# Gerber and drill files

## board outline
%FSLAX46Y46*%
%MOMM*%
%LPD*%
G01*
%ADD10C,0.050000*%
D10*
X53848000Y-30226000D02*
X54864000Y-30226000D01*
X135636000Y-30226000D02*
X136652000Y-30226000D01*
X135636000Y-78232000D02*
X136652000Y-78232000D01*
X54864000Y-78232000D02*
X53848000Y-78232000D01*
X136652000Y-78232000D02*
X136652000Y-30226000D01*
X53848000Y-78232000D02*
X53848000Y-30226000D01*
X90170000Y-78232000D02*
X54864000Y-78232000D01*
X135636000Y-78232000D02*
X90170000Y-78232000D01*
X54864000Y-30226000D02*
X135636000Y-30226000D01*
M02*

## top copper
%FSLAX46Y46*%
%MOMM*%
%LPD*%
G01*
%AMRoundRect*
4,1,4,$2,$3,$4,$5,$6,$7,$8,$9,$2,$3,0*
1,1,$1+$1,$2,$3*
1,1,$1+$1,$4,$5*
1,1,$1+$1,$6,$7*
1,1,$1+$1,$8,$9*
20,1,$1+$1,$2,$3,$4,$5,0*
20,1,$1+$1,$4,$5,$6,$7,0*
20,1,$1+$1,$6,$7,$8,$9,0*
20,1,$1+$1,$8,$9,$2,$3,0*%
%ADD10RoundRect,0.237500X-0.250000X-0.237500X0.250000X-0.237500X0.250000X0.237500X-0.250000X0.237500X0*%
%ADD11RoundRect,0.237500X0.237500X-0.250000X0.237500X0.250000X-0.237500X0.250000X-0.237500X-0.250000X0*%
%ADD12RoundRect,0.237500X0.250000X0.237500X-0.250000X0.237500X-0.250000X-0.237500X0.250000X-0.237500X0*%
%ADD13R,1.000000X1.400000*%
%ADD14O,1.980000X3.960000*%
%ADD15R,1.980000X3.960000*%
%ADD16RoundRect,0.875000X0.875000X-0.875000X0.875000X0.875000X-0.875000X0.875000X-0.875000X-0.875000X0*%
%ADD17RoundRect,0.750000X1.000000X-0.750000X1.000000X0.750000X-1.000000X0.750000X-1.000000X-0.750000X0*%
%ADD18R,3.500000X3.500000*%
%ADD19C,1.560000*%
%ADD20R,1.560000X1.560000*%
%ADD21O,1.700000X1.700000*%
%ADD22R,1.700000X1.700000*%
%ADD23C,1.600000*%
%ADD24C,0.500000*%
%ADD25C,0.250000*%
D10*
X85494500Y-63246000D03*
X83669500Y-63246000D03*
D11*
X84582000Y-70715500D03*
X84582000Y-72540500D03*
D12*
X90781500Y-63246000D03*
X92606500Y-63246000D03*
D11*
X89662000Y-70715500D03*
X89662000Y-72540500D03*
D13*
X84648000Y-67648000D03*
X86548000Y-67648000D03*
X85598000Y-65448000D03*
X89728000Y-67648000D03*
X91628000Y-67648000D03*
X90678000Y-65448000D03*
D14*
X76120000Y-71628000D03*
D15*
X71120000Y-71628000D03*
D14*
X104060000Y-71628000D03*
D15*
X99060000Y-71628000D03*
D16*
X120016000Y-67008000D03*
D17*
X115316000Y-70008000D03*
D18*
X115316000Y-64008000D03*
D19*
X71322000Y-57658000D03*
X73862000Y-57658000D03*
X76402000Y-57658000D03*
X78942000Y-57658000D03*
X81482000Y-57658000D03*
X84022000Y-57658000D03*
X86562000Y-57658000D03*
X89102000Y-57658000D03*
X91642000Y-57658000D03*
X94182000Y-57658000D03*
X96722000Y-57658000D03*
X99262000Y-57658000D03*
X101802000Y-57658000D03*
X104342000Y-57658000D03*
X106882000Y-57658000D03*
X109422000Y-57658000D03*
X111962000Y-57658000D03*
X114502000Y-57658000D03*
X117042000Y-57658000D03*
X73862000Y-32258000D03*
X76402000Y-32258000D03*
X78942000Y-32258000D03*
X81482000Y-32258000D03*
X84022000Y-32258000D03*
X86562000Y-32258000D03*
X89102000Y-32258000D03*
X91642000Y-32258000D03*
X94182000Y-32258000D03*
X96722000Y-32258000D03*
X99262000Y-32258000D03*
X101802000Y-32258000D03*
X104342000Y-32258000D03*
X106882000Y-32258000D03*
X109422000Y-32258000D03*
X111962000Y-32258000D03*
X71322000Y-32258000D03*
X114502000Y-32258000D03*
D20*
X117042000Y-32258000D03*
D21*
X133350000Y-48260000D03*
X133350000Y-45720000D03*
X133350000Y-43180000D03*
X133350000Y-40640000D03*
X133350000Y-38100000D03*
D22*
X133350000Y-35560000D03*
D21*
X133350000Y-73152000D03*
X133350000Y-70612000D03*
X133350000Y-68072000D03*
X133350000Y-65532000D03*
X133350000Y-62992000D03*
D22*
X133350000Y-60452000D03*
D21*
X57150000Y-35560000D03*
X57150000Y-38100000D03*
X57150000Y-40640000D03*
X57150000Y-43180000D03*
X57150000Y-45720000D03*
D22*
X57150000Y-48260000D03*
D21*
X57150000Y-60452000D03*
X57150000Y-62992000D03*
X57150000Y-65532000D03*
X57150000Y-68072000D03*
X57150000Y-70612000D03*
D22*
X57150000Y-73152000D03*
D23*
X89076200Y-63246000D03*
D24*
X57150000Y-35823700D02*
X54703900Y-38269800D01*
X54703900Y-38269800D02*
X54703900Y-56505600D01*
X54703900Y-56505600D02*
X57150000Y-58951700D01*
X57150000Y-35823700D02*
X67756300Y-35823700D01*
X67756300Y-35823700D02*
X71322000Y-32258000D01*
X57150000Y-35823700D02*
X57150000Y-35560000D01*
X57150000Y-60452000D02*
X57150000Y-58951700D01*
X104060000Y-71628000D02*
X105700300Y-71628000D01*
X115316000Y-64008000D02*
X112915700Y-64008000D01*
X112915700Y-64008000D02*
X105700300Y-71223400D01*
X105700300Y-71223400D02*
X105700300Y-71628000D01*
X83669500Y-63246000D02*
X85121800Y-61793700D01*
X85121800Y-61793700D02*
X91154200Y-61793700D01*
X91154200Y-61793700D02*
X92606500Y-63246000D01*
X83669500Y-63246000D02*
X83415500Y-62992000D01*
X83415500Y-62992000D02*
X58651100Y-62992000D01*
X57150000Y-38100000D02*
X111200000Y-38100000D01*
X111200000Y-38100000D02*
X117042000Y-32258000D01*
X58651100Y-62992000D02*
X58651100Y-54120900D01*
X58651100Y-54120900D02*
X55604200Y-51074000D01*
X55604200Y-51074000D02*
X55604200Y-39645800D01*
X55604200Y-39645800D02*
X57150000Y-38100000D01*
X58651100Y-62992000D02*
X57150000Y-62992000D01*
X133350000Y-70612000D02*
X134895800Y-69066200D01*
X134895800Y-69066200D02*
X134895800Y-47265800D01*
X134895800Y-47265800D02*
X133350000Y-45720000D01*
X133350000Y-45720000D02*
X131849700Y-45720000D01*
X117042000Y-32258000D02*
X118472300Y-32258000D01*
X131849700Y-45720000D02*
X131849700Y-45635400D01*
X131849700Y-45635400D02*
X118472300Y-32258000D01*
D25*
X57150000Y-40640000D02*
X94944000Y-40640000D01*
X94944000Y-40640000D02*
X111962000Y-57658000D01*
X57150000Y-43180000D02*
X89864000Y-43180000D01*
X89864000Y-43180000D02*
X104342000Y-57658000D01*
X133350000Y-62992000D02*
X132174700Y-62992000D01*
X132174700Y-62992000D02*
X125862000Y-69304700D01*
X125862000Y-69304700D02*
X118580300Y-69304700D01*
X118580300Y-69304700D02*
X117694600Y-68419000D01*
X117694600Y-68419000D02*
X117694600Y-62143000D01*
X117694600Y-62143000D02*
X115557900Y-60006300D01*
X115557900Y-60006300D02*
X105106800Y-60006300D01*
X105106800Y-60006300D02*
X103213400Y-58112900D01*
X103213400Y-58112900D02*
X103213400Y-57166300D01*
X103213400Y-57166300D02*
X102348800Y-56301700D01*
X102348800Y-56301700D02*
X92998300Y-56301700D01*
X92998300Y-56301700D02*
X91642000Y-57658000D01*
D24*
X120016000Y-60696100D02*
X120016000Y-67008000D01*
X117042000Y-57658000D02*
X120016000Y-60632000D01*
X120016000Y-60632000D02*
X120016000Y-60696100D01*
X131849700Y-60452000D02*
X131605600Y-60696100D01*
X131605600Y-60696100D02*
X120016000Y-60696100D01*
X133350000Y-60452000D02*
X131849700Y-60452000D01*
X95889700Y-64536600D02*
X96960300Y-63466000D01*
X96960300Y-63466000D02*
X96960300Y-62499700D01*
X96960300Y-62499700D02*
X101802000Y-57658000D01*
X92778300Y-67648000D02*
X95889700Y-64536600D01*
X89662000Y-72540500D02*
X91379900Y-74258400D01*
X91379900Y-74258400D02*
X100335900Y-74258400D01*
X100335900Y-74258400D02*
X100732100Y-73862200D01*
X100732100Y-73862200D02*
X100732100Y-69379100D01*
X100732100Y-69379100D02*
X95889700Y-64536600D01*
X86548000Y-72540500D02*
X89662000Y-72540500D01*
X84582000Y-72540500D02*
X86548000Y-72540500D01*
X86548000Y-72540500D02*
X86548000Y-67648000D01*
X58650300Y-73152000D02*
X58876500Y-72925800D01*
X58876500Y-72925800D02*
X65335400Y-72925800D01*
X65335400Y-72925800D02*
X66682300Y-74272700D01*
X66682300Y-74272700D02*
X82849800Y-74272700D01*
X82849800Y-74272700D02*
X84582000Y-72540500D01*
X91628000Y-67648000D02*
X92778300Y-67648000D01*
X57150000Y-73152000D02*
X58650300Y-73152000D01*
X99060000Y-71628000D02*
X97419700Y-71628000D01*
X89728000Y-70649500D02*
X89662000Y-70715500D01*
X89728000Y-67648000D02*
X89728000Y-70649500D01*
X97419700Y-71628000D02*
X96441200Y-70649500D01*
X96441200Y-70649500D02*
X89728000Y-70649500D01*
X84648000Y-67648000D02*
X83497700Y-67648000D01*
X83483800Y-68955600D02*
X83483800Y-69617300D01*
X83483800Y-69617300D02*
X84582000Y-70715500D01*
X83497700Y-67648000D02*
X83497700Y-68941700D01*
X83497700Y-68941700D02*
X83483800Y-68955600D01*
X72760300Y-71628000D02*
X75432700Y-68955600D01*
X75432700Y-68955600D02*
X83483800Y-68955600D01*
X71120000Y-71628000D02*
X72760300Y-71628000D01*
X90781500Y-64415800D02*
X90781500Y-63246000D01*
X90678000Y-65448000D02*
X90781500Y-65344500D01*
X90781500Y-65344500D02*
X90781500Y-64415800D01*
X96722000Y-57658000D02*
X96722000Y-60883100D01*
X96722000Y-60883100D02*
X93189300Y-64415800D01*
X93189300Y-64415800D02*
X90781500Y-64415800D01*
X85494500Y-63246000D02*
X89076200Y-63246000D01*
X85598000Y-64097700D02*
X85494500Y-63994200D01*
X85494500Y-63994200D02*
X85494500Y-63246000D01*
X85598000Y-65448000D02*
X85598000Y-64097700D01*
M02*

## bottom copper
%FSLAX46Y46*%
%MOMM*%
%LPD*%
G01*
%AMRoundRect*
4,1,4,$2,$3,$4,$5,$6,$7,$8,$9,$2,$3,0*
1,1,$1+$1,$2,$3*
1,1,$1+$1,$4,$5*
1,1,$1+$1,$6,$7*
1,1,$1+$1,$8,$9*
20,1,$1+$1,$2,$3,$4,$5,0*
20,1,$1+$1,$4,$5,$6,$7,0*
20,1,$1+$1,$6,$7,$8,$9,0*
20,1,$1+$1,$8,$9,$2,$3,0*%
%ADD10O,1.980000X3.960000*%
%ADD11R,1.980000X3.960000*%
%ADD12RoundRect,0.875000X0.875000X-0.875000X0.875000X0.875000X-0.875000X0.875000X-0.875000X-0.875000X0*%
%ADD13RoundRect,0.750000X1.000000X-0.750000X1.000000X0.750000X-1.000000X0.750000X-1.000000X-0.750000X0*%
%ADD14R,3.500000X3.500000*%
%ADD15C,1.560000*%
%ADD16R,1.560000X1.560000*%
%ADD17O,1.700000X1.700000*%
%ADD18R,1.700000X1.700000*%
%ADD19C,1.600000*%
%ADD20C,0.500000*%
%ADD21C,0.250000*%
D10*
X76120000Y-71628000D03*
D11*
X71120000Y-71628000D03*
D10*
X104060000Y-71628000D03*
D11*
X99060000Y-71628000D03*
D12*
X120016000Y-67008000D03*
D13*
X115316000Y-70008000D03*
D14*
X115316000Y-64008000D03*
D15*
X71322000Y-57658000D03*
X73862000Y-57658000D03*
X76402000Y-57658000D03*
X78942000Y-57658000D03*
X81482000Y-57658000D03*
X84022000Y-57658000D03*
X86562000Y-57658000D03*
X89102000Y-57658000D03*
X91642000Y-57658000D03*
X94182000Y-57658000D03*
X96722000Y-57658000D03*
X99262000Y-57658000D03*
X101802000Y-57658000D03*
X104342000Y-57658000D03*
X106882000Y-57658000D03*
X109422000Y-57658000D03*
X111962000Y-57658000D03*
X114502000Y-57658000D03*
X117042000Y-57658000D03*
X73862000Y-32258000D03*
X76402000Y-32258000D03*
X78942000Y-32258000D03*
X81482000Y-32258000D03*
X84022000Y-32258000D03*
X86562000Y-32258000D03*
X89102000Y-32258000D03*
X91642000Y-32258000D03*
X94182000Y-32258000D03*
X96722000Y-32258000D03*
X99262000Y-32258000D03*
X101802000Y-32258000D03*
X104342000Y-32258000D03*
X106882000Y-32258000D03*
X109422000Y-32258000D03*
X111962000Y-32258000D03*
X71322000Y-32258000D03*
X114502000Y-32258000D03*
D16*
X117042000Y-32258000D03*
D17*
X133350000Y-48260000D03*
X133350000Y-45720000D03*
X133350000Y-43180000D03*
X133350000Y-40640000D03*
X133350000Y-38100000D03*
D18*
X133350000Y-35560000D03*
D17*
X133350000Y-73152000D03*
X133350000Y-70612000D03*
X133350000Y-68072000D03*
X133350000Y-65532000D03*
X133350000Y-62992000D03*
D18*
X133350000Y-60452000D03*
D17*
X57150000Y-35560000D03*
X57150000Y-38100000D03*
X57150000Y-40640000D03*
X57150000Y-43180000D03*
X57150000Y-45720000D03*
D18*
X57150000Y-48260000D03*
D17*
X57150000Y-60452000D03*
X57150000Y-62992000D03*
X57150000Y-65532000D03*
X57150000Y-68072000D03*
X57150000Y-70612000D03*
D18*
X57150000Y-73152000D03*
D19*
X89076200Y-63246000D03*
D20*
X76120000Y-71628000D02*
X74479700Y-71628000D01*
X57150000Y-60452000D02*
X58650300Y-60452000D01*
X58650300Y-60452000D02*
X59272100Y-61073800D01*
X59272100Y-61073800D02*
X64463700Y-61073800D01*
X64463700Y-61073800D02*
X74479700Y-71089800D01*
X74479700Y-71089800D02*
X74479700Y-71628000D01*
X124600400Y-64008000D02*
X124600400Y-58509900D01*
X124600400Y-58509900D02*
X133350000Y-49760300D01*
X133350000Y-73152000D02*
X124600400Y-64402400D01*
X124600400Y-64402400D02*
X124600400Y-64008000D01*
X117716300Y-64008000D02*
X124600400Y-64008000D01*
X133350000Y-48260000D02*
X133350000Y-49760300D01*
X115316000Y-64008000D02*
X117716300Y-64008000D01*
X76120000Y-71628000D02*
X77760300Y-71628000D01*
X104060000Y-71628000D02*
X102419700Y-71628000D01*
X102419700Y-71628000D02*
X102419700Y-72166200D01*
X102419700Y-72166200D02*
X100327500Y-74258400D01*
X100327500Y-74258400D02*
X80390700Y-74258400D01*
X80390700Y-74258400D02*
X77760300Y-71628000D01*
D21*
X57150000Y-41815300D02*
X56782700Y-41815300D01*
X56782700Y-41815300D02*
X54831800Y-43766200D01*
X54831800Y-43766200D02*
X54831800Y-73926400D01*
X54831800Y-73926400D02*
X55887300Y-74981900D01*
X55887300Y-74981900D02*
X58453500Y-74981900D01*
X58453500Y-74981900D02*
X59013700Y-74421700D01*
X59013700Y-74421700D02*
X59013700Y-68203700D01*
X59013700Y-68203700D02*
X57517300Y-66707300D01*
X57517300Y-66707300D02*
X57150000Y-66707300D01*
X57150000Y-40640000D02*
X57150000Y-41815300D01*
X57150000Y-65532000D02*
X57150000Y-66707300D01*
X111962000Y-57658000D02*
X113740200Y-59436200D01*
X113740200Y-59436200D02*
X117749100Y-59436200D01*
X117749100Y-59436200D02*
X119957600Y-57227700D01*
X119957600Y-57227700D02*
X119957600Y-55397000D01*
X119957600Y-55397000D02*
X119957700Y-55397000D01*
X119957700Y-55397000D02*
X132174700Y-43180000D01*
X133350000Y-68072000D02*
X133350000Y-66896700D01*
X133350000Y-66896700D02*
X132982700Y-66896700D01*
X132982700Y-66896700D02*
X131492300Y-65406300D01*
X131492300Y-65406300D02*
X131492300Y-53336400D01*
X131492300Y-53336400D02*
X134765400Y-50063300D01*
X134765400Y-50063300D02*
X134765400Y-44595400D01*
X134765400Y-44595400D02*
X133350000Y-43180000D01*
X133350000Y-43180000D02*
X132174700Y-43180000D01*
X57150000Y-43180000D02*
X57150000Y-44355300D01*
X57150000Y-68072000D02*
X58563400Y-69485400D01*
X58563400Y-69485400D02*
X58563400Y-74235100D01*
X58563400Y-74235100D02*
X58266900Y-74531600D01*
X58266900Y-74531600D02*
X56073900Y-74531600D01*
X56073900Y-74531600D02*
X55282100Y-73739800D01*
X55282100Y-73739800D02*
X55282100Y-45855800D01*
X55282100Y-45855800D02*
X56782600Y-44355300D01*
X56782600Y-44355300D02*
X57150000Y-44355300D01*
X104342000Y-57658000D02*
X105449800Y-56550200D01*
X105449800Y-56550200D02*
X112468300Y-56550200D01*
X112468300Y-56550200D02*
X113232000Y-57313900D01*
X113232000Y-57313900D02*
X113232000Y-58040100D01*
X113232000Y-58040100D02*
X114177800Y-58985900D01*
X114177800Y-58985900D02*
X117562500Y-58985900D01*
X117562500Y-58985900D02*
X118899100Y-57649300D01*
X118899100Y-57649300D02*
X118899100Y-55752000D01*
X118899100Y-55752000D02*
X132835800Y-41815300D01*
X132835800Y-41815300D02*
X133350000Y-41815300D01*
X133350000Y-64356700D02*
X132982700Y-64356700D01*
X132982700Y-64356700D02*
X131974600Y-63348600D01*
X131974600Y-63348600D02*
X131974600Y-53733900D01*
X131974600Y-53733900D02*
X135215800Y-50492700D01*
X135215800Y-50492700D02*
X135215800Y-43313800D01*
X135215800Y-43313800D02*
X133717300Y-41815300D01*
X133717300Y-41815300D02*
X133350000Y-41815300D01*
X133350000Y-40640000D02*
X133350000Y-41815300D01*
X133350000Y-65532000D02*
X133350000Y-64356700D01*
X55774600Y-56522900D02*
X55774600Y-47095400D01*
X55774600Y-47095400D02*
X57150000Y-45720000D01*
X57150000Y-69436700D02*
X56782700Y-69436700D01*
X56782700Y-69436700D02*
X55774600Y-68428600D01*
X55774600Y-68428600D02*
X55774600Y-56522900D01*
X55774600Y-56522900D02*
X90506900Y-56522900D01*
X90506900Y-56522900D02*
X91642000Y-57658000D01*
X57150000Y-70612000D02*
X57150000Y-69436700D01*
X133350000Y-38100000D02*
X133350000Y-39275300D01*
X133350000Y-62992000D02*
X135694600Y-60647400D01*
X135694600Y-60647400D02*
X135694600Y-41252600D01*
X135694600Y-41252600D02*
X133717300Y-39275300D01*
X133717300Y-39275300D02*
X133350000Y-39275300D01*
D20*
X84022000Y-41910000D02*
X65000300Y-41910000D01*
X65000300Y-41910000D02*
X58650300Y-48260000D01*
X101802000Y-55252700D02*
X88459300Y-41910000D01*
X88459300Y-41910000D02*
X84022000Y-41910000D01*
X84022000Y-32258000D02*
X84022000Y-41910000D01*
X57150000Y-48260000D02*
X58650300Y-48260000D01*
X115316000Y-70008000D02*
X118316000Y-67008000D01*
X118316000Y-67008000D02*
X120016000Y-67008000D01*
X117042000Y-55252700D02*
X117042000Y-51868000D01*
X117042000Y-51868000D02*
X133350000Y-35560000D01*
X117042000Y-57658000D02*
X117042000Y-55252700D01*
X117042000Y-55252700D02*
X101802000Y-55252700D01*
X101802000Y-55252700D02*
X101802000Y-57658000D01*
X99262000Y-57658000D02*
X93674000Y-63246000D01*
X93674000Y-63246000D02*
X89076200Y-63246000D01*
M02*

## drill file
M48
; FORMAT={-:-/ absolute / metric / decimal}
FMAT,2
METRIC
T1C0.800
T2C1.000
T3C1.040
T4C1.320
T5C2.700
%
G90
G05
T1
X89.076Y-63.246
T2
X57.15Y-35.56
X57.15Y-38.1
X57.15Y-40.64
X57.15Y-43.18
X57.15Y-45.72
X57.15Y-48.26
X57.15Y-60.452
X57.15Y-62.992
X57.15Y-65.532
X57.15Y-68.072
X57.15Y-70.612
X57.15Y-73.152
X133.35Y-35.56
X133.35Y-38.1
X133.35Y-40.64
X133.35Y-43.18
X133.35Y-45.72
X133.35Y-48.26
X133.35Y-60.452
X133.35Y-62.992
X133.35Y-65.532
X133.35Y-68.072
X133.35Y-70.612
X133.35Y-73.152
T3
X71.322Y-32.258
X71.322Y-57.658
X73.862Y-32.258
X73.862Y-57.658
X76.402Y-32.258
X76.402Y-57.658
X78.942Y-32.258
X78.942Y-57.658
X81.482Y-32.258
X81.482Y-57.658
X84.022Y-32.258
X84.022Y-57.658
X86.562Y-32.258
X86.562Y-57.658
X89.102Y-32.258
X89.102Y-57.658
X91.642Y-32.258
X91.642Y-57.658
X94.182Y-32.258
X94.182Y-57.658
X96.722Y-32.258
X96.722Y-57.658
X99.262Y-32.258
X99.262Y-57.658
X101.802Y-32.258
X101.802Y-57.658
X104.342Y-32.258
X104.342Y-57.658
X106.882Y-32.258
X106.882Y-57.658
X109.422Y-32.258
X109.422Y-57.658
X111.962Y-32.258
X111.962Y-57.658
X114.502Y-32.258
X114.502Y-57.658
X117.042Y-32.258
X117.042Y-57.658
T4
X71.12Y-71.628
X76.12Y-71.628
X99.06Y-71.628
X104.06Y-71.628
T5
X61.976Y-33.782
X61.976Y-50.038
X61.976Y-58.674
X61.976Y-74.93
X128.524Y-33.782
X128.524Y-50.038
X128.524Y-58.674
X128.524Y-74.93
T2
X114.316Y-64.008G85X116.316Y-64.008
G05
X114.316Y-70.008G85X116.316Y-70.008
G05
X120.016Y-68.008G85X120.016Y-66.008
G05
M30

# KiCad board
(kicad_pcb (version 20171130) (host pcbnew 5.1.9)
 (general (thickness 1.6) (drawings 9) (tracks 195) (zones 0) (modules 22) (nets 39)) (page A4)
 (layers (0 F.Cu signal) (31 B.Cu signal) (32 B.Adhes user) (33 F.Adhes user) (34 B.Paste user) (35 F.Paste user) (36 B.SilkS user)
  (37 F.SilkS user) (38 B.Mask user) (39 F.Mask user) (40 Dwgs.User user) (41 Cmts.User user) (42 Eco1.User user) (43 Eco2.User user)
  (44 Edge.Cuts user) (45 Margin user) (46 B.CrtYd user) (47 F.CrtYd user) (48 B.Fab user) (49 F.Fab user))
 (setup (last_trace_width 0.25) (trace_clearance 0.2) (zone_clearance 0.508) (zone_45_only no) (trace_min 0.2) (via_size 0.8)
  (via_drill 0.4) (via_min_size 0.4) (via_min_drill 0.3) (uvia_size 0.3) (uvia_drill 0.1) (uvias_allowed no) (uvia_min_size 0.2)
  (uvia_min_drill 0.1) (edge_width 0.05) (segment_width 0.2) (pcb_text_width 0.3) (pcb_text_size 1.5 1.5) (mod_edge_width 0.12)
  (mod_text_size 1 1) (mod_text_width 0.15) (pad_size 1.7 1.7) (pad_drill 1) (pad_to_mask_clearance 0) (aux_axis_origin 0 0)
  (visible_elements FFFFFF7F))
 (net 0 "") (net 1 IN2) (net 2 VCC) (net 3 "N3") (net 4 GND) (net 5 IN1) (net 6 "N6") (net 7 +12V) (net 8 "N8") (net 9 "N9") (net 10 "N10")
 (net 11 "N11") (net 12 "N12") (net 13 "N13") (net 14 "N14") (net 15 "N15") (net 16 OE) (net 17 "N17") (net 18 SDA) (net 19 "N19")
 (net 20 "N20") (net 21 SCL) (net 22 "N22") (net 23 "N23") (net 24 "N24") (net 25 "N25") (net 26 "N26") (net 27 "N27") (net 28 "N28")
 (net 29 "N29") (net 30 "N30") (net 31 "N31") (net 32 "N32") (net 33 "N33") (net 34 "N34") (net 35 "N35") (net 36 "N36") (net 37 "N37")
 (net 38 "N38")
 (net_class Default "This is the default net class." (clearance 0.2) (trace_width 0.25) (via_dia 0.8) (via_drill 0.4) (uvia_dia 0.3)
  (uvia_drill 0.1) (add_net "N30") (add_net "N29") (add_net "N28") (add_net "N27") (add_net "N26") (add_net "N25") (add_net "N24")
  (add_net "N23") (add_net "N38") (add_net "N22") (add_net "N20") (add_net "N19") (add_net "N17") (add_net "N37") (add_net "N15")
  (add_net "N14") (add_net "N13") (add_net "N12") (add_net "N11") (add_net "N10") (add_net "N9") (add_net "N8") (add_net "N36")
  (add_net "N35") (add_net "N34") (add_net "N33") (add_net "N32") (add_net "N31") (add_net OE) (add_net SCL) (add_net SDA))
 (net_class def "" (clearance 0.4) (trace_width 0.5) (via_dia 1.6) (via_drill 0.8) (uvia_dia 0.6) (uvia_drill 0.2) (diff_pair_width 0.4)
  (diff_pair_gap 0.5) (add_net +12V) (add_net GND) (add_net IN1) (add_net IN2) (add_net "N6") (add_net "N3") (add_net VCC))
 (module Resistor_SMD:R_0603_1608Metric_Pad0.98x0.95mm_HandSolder (layer F.Cu) (at 84.582 63.246)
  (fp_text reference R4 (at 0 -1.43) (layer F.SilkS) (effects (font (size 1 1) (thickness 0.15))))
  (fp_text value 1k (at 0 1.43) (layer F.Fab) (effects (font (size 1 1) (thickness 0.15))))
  (pad 2 smd roundrect (at 0.9125 0) (size 0.975 0.95) (layers F.Cu F.Paste F.Mask) (roundrect_rratio 0.25) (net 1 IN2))
  (pad 1 smd roundrect (at -0.9125 0) (size 0.975 0.95) (layers F.Cu F.Paste F.Mask) (roundrect_rratio 0.25) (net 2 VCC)))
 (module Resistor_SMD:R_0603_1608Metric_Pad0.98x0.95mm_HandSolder (layer F.Cu) (at 84.582 71.628 90)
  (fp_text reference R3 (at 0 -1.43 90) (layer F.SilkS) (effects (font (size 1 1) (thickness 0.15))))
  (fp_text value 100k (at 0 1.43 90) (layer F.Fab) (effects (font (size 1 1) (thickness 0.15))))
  (pad 2 smd roundrect (at 0.9125 0 90) (size 0.975 0.95) (layers F.Cu F.Paste F.Mask) (roundrect_rratio 0.25) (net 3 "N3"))
  (pad 1 smd roundrect (at -0.9125 0 90) (size 0.975 0.95) (layers F.Cu F.Paste F.Mask) (roundrect_rratio 0.25) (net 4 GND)))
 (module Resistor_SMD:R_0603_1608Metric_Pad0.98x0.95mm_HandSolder (layer F.Cu) (at 91.694 63.246 180)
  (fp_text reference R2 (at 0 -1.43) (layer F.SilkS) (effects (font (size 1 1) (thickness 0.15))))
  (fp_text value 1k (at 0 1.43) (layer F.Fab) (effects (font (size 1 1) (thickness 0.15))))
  (pad 2 smd roundrect (at 0.9125 0 180) (size 0.975 0.95) (layers F.Cu F.Paste F.Mask) (roundrect_rratio 0.25) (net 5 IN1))
  (pad 1 smd roundrect (at -0.9125 0 180) (size 0.975 0.95) (layers F.Cu F.Paste F.Mask) (roundrect_rratio 0.25) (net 2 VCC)))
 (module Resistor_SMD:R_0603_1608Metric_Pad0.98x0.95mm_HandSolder (layer F.Cu) (at 89.662 71.628 90)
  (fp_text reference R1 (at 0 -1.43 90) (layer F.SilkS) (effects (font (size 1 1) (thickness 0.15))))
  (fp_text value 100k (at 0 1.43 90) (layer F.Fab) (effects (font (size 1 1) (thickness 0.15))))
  (pad 2 smd roundrect (at 0.9125 0 90) (size 0.975 0.95) (layers F.Cu F.Paste F.Mask) (roundrect_rratio 0.25) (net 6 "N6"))
  (pad 1 smd roundrect (at -0.9125 0 90) (size 0.975 0.95) (layers F.Cu F.Paste F.Mask) (roundrect_rratio 0.25) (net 4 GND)))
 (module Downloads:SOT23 (layer F.Cu) (at 85.598 66.548)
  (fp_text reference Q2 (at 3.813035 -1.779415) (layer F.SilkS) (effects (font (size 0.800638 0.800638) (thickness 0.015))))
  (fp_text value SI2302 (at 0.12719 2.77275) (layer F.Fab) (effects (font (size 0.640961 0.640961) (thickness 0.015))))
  (pad 1 smd rect (at -0.95 1.1) (size 1 1.4) (layers F.Cu F.Paste F.Mask) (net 3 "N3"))
  (pad 2 smd rect (at 0.95 1.1) (size 1 1.4) (layers F.Cu F.Paste F.Mask) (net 4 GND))
  (pad 3 smd rect (at 0 -1.1) (size 1 1.4) (layers F.Cu F.Paste F.Mask) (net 1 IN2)))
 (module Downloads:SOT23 (layer F.Cu) (at 90.678 66.548)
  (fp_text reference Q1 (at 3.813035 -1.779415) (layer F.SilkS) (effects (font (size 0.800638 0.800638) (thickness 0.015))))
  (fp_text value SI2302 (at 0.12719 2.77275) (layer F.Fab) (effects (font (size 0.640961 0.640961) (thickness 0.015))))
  (pad 1 smd rect (at -0.95 1.1) (size 1 1.4) (layers F.Cu F.Paste F.Mask) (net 6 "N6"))
  (pad 2 smd rect (at 0.95 1.1) (size 1 1.4) (layers F.Cu F.Paste F.Mask) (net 4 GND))
  (pad 3 smd rect (at 0 -1.1) (size 1 1.4) (layers F.Cu F.Paste F.Mask) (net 5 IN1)))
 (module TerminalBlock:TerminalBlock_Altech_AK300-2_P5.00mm (layer F.Cu) (at 71.12 71.628)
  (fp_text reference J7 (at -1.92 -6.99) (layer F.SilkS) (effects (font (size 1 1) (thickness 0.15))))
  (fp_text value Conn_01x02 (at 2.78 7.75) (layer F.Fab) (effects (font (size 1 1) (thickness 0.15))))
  (pad 2 thru_hole oval (at 5 0) (size 1.98 3.96) (drill 1.32) (layers *.Cu *.Mask) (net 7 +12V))
  (pad 1 thru_hole rect (at 0 0) (size 1.98 3.96) (drill 1.32) (layers *.Cu *.Mask) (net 3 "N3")))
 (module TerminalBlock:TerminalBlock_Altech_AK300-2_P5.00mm (layer F.Cu) (at 99.06 71.628)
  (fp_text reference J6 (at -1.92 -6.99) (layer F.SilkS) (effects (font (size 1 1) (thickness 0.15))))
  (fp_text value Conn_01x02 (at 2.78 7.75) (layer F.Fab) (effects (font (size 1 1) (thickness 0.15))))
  (pad 2 thru_hole oval (at 5 0) (size 1.98 3.96) (drill 1.32) (layers *.Cu *.Mask) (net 7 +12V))
  (pad 1 thru_hole rect (at 0 0) (size 1.98 3.96) (drill 1.32) (layers *.Cu *.Mask) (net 6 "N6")))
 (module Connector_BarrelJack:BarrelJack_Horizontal (layer F.Cu) (at 115.316 64.008 90)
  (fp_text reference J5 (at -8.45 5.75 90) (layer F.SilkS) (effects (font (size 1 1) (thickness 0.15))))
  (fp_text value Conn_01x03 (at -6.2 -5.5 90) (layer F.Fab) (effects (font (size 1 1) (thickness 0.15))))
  (pad 3 thru_hole roundrect (at -3 4.7 90) (size 3.5 3.5) (drill oval 3 1) (layers *.Cu *.Mask) (roundrect_rratio 0.25) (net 4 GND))
  (pad 2 thru_hole roundrect (at -6 0 90) (size 3 3.5) (drill oval 1 3) (layers *.Cu *.Mask) (roundrect_rratio 0.25) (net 4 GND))
  (pad 1 thru_hole rect (at 0 0 90) (size 3.5 3.5) (drill oval 1 3) (layers *.Cu *.Mask) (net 7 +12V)))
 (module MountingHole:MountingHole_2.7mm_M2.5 (layer F.Cu) (at 128.524 74.93)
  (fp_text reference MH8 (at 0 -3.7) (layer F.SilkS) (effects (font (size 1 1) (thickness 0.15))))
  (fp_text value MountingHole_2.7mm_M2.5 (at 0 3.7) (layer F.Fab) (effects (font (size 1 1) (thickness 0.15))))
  (pad 1 np_thru_hole circle (at 0 0) (size 2.7 2.7) (drill 2.7) (layers *.Cu *.Mask)))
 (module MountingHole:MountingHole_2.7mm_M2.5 (layer F.Cu) (at 128.524 58.674)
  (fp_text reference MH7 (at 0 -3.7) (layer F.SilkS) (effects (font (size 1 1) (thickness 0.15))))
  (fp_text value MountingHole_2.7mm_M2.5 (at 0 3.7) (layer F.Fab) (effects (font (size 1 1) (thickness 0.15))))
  (pad 1 np_thru_hole circle (at 0 0) (size 2.7 2.7) (drill 2.7) (layers *.Cu *.Mask)))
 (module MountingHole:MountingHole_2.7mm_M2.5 (layer F.Cu) (at 128.524 50.038)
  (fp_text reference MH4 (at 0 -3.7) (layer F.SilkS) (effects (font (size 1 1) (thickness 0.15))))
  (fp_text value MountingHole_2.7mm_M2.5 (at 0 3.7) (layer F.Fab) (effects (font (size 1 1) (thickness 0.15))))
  (pad 1 np_thru_hole circle (at 0 0) (size 2.7 2.7) (drill 2.7) (layers *.Cu *.Mask)))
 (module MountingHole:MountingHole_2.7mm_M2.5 (layer F.Cu) (at 128.524 33.782)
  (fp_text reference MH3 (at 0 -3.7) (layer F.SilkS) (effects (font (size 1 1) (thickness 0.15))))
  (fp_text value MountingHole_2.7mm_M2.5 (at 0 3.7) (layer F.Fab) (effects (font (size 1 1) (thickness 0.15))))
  (pad 1 np_thru_hole circle (at 0 0) (size 2.7 2.7) (drill 2.7) (layers *.Cu *.Mask)))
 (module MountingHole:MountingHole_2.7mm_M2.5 (layer F.Cu) (at 61.976 74.93)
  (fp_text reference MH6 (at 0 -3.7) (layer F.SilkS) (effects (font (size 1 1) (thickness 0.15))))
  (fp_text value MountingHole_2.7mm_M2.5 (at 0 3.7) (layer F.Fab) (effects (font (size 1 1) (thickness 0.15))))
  (pad 1 np_thru_hole circle (at 0 0) (size 2.7 2.7) (drill 2.7) (layers *.Cu *.Mask)))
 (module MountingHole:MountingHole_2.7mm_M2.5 (layer F.Cu) (at 61.976 58.674)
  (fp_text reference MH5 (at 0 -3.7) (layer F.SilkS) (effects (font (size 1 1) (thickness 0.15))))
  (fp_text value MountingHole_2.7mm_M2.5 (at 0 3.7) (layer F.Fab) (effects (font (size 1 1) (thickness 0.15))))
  (pad 1 np_thru_hole circle (at 0 0) (size 2.7 2.7) (drill 2.7) (layers *.Cu *.Mask)))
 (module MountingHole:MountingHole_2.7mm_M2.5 (layer F.Cu) (at 61.976 50.038)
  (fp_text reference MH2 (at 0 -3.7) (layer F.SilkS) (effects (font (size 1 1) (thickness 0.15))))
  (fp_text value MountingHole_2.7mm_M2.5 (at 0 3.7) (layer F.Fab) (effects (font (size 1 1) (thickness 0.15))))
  (pad 1 np_thru_hole circle (at 0 0) (size 2.7 2.7) (drill 2.7) (layers *.Cu *.Mask)))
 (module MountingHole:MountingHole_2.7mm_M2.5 (layer F.Cu) (at 61.976 33.782)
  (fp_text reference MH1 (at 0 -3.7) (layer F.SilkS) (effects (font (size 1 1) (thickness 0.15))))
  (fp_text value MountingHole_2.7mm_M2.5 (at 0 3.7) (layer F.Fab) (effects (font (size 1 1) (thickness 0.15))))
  (pad 1 np_thru_hole circle (at 0 0) (size 2.7 2.7) (drill 2.7) (layers *.Cu *.Mask)))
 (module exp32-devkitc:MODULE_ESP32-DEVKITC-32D (layer F.Cu) (at 97.282 44.958 270)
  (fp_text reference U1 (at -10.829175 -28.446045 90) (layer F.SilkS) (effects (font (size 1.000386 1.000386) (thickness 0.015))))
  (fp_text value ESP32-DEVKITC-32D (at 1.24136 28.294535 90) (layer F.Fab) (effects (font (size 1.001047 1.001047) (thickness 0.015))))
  (pad 38 thru_hole circle (at 12.7 25.96 270) (size 1.56 1.56) (drill 1.04) (layers *.Cu *.Mask) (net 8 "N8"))
  (pad 37 thru_hole circle (at 12.7 23.42 270) (size 1.56 1.56) (drill 1.04) (layers *.Cu *.Mask) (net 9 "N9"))
  (pad 36 thru_hole circle (at 12.7 20.88 270) (size 1.56 1.56) (drill 1.04) (layers *.Cu *.Mask) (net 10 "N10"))
  (pad 35 thru_hole circle (at 12.7 18.34 270) (size 1.56 1.56) (drill 1.04) (layers *.Cu *.Mask) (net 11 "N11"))
  (pad 34 thru_hole circle (at 12.7 15.8 270) (size 1.56 1.56) (drill 1.04) (layers *.Cu *.Mask) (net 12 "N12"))
  (pad 33 thru_hole circle (at 12.7 13.26 270) (size 1.56 1.56) (drill 1.04) (layers *.Cu *.Mask) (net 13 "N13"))
  (pad 32 thru_hole circle (at 12.7 10.72 270) (size 1.56 1.56) (drill 1.04) (layers *.Cu *.Mask) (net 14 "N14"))
  (pad 31 thru_hole circle (at 12.7 8.18 270) (size 1.56 1.56) (drill 1.04) (layers *.Cu *.Mask) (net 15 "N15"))
  (pad 30 thru_hole circle (at 12.7 5.64 270) (size 1.56 1.56) (drill 1.04) (layers *.Cu *.Mask) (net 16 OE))
  (pad 29 thru_hole circle (at 12.7 3.1 270) (size 1.56 1.56) (drill 1.04) (layers *.Cu *.Mask) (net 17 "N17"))
  (pad 28 thru_hole circle (at 12.7 0.56 270) (size 1.56 1.56) (drill 1.04) (layers *.Cu *.Mask) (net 5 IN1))
  (pad 27 thru_hole circle (at 12.7 -1.98 270) (size 1.56 1.56) (drill 1.04) (layers *.Cu *.Mask) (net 1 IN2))
  (pad 26 thru_hole circle (at 12.7 -4.52 270) (size 1.56 1.56) (drill 1.04) (layers *.Cu *.Mask) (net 4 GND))
  (pad 25 thru_hole circle (at 12.7 -7.06 270) (size 1.56 1.56) (drill 1.04) (layers *.Cu *.Mask) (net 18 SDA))
  (pad 24 thru_hole circle (at 12.7 -9.6 270) (size 1.56 1.56) (drill 1.04) (layers *.Cu *.Mask) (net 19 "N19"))
  (pad 23 thru_hole circle (at 12.7 -12.14 270) (size 1.56 1.56) (drill 1.04) (layers *.Cu *.Mask) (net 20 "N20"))
  (pad 22 thru_hole circle (at 12.7 -14.68 270) (size 1.56 1.56) (drill 1.04) (layers *.Cu *.Mask) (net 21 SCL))
  (pad 21 thru_hole circle (at 12.7 -17.22 270) (size 1.56 1.56) (drill 1.04) (layers *.Cu *.Mask) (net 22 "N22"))
  (pad 20 thru_hole circle (at 12.7 -19.76 270) (size 1.56 1.56) (drill 1.04) (layers *.Cu *.Mask) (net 4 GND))
  (pad 18 thru_hole circle (at -12.7 23.42 270) (size 1.56 1.56) (drill 1.04) (layers *.Cu *.Mask) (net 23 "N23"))
  (pad 17 thru_hole circle (at -12.7 20.88 270) (size 1.56 1.56) (drill 1.04) (layers *.Cu *.Mask) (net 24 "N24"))
  (pad 16 thru_hole circle (at -12.7 18.34 270) (size 1.56 1.56) (drill 1.04) (layers *.Cu *.Mask) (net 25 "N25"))
  (pad 15 thru_hole circle (at -12.7 15.8 270) (size 1.56 1.56) (drill 1.04) (layers *.Cu *.Mask) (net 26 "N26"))
  (pad 14 thru_hole circle (at -12.7 13.26 270) (size 1.56 1.56) (drill 1.04) (layers *.Cu *.Mask) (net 4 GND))
  (pad 13 thru_hole circle (at -12.7 10.72 270) (size 1.56 1.56) (drill 1.04) (layers *.Cu *.Mask) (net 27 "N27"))
  (pad 12 thru_hole circle (at -12.7 8.18 270) (size 1.56 1.56) (drill 1.04) (layers *.Cu *.Mask) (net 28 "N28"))
  (pad 11 thru_hole circle (at -12.7 5.64 270) (size 1.56 1.56) (drill 1.04) (layers *.Cu *.Mask) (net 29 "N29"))
  (pad 10 thru_hole circle (at -12.7 3.1 270) (size 1.56 1.56) (drill 1.04) (layers *.Cu *.Mask) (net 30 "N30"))
  (pad 9 thru_hole circle (at -12.7 0.56 270) (size 1.56 1.56) (drill 1.04) (layers *.Cu *.Mask) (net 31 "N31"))
  (pad 8 thru_hole circle (at -12.7 -1.98 270) (size 1.56 1.56) (drill 1.04) (layers *.Cu *.Mask) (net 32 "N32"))
  (pad 7 thru_hole circle (at -12.7 -4.52 270) (size 1.56 1.56) (drill 1.04) (layers *.Cu *.Mask) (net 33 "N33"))
  (pad 6 thru_hole circle (at -12.7 -7.06 270) (size 1.56 1.56) (drill 1.04) (layers *.Cu *.Mask) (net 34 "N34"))
  (pad 5 thru_hole circle (at -12.7 -9.6 270) (size 1.56 1.56) (drill 1.04) (layers *.Cu *.Mask) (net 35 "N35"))
  (pad 4 thru_hole circle (at -12.7 -12.14 270) (size 1.56 1.56) (drill 1.04) (layers *.Cu *.Mask) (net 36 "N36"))
  (pad 3 thru_hole circle (at -12.7 -14.68 270) (size 1.56 1.56) (drill 1.04) (layers *.Cu *.Mask) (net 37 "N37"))
  (pad 19 thru_hole circle (at -12.7 25.96 270) (size 1.56 1.56) (drill 1.04) (layers *.Cu *.Mask) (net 7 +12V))
  (pad 2 thru_hole circle (at -12.7 -17.22 270) (size 1.56 1.56) (drill 1.04) (layers *.Cu *.Mask) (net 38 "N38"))
  (pad 1 thru_hole rect (at -12.7 -19.76 270) (size 1.56 1.56) (drill 1.04) (layers *.Cu *.Mask) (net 2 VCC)))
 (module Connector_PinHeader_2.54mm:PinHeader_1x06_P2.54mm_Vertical (layer F.Cu) (at 133.35 35.56)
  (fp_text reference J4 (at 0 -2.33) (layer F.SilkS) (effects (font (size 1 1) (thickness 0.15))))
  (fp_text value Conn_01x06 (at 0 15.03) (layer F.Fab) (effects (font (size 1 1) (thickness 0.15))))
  (pad 6 thru_hole oval (at 0 12.7) (size 1.7 1.7) (drill 1) (layers *.Cu *.Mask) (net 7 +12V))
  (pad 5 thru_hole oval (at 0 10.16) (size 1.7 1.7) (drill 1) (layers *.Cu *.Mask) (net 2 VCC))
  (pad 4 thru_hole oval (at 0 7.62) (size 1.7 1.7) (drill 1) (layers *.Cu *.Mask) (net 21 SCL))
  (pad 3 thru_hole oval (at 0 5.08) (size 1.7 1.7) (drill 1) (layers *.Cu *.Mask) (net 18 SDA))
  (pad 2 thru_hole oval (at 0 2.54) (size 1.7 1.7) (drill 1) (layers *.Cu *.Mask) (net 16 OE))
  (pad 1 thru_hole rect (at 0 0) (size 1.7 1.7) (drill 1) (layers *.Cu *.Mask) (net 4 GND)))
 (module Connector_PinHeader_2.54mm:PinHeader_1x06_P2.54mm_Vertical (layer F.Cu) (at 133.35 60.452)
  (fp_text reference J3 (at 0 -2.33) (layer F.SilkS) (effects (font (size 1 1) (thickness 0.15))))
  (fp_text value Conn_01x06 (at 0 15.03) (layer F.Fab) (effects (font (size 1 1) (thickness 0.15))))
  (pad 6 thru_hole oval (at 0 12.7) (size 1.7 1.7) (drill 1) (layers *.Cu *.Mask) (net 7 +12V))
  (pad 5 thru_hole oval (at 0 10.16) (size 1.7 1.7) (drill 1) (layers *.Cu *.Mask) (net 2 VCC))
  (pad 4 thru_hole oval (at 0 7.62) (size 1.7 1.7) (drill 1) (layers *.Cu *.Mask) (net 21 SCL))
  (pad 3 thru_hole oval (at 0 5.08) (size 1.7 1.7) (drill 1) (layers *.Cu *.Mask) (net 18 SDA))
  (pad 2 thru_hole oval (at 0 2.54) (size 1.7 1.7) (drill 1) (layers *.Cu *.Mask) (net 16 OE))
  (pad 1 thru_hole rect (at 0 0) (size 1.7 1.7) (drill 1) (layers *.Cu *.Mask) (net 4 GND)))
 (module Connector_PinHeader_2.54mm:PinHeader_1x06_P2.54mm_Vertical (layer F.Cu) (at 57.15 48.26 180)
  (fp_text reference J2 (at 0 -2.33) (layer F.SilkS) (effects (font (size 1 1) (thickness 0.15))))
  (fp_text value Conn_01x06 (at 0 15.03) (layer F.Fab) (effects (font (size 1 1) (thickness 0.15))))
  (pad 6 thru_hole oval (at 0 12.7 180) (size 1.7 1.7) (drill 1) (layers *.Cu *.Mask) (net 7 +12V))
  (pad 5 thru_hole oval (at 0 10.16 180) (size 1.7 1.7) (drill 1) (layers *.Cu *.Mask) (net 2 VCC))
  (pad 4 thru_hole oval (at 0 7.62 180) (size 1.7 1.7) (drill 1) (layers *.Cu *.Mask) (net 21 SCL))
  (pad 3 thru_hole oval (at 0 5.08 180) (size 1.7 1.7) (drill 1) (layers *.Cu *.Mask) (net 18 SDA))
  (pad 2 thru_hole oval (at 0 2.54 180) (size 1.7 1.7) (drill 1) (layers *.Cu *.Mask) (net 16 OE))
  (pad 1 thru_hole rect (at 0 0 180) (size 1.7 1.7) (drill 1) (layers *.Cu *.Mask) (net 4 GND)))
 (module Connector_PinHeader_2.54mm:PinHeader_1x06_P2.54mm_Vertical (layer F.Cu) (at 57.15 73.152 180)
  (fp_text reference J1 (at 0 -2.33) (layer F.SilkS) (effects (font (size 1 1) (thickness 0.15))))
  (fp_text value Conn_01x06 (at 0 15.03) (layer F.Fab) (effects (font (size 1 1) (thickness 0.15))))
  (pad 6 thru_hole oval (at 0 12.7 180) (size 1.7 1.7) (drill 1) (layers *.Cu *.Mask) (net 7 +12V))
  (pad 5 thru_hole oval (at 0 10.16 180) (size 1.7 1.7) (drill 1) (layers *.Cu *.Mask) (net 2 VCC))
  (pad 4 thru_hole oval (at 0 7.62 180) (size 1.7 1.7) (drill 1) (layers *.Cu *.Mask) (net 21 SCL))
  (pad 3 thru_hole oval (at 0 5.08 180) (size 1.7 1.7) (drill 1) (layers *.Cu *.Mask) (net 18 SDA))
  (pad 2 thru_hole oval (at 0 2.54 180) (size 1.7 1.7) (drill 1) (layers *.Cu *.Mask) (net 16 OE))
  (pad 1 thru_hole rect (at 0 0 180) (size 1.7 1.7) (drill 1) (layers *.Cu *.Mask) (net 4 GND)))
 (gr_line (start 53.848 30.226) (end 54.864 30.226) (layer Edge.Cuts) (width 0.05))
 (gr_line (start 135.636 30.226) (end 136.652 30.226) (layer Edge.Cuts) (width 0.05))
 (gr_line (start 135.636 78.232) (end 136.652 78.232) (layer Edge.Cuts) (width 0.05))
 (gr_line (start 54.864 78.232) (end 53.848 78.232) (layer Edge.Cuts) (width 0.05))
 (gr_line (start 136.652 78.232) (end 136.652 30.226) (layer Edge.Cuts) (width 0.05))
 (gr_line (start 53.848 78.232) (end 53.848 30.226) (layer Edge.Cuts) (width 0.05))
 (gr_line (start 90.17 78.232) (end 54.864 78.232) (layer Edge.Cuts) (width 0.05))
 (gr_line (start 135.636 78.232) (end 90.17 78.232) (layer Edge.Cuts) (width 0.05))
 (gr_line (start 54.864 30.226) (end 135.636 30.226) (layer Edge.Cuts) (width 0.05))
 (segment (start 76.12 71.628) (end 74.4797 71.628) (width 0.5) (layer B.Cu) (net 7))
 (segment (start 57.15 60.452) (end 58.6503 60.452) (width 0.5) (layer B.Cu) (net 7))
 (segment (start 58.6503 60.452) (end 59.2721 61.0738) (width 0.5) (layer B.Cu) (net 7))
 (segment (start 59.2721 61.0738) (end 64.4637 61.0738) (width 0.5) (layer B.Cu) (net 7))
 (segment (start 64.4637 61.0738) (end 74.4797 71.0898) (width 0.5) (layer B.Cu) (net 7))
 (segment (start 74.4797 71.0898) (end 74.4797 71.628) (width 0.5) (layer B.Cu) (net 7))
 (segment (start 57.15 35.8237) (end 54.7039 38.2698) (width 0.5) (layer F.Cu) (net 7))
 (segment (start 54.7039 38.2698) (end 54.7039 56.5056) (width 0.5) (layer F.Cu) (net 7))
 (segment (start 54.7039 56.5056) (end 57.15 58.9517) (width 0.5) (layer F.Cu) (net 7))
 (segment (start 124.6004 64.008) (end 124.6004 58.5099) (width 0.5) (layer B.Cu) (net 7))
 (segment (start 124.6004 58.5099) (end 133.35 49.7603) (width 0.5) (layer B.Cu) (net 7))
 (segment (start 133.35 73.152) (end 124.6004 64.4024) (width 0.5) (layer B.Cu) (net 7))
 (segment (start 124.6004 64.4024) (end 124.6004 64.008) (width 0.5) (layer B.Cu) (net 7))
 (segment (start 117.7163 64.008) (end 124.6004 64.008) (width 0.5) (layer B.Cu) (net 7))
 (segment (start 133.35 48.26) (end 133.35 49.7603) (width 0.5) (layer B.Cu) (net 7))
 (segment (start 115.316 64.008) (end 117.7163 64.008) (width 0.5) (layer B.Cu) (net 7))
 (segment (start 57.15 35.8237) (end 67.7563 35.8237) (width 0.5) (layer F.Cu) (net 7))
 (segment (start 67.7563 35.8237) (end 71.322 32.258) (width 0.5) (layer F.Cu) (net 7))
 (segment (start 57.15 35.8237) (end 57.15 35.56) (width 0.5) (layer F.Cu) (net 7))
 (segment (start 57.15 60.452) (end 57.15 58.9517) (width 0.5) (layer F.Cu) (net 7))
 (segment (start 76.12 71.628) (end 77.7603 71.628) (width 0.5) (layer B.Cu) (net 7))
 (segment (start 104.06 71.628) (end 102.4197 71.628) (width 0.5) (layer B.Cu) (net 7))
 (segment (start 102.4197 71.628) (end 102.4197 72.1662) (width 0.5) (layer B.Cu) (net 7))
 (segment (start 102.4197 72.1662) (end 100.3275 74.2584) (width 0.5) (layer B.Cu) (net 7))
 (segment (start 100.3275 74.2584) (end 80.3907 74.2584) (width 0.5) (layer B.Cu) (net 7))
 (segment (start 80.3907 74.2584) (end 77.7603 71.628) (width 0.5) (layer B.Cu) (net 7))
 (segment (start 104.06 71.628) (end 105.7003 71.628) (width 0.5) (layer F.Cu) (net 7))
 (segment (start 115.316 64.008) (end 112.9157 64.008) (width 0.5) (layer F.Cu) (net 7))
 (segment (start 112.9157 64.008) (end 105.7003 71.2234) (width 0.5) (layer F.Cu) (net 7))
 (segment (start 105.7003 71.2234) (end 105.7003 71.628) (width 0.5) (layer F.Cu) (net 7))
 (segment (start 83.6695 63.246) (end 85.1218 61.7937) (width 0.5) (layer F.Cu) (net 2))
 (segment (start 85.1218 61.7937) (end 91.1542 61.7937) (width 0.5) (layer F.Cu) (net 2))
 (segment (start 91.1542 61.7937) (end 92.6065 63.246) (width 0.5) (layer F.Cu) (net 2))
 (segment (start 83.6695 63.246) (end 83.4155 62.992) (width 0.5) (layer F.Cu) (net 2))
 (segment (start 83.4155 62.992) (end 58.6511 62.992) (width 0.5) (layer F.Cu) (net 2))
 (segment (start 57.15 38.1) (end 111.2 38.1) (width 0.5) (layer F.Cu) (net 2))
 (segment (start 111.2 38.1) (end 117.042 32.258) (width 0.5) (layer F.Cu) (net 2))
 (segment (start 58.6511 62.992) (end 58.6511 54.1209) (width 0.5) (layer F.Cu) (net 2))
 (segment (start 58.6511 54.1209) (end 55.6042 51.074) (width 0.5) (layer F.Cu) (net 2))
 (segment (start 55.6042 51.074) (end 55.6042 39.6458) (width 0.5) (layer F.Cu) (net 2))
 (segment (start 55.6042 39.6458) (end 57.15 38.1) (width 0.5) (layer F.Cu) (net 2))
 (segment (start 58.6511 62.992) (end 57.15 62.992) (width 0.5) (layer F.Cu) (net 2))
 (segment (start 133.35 70.612) (end 134.8958 69.0662) (width 0.5) (layer F.Cu) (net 2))
 (segment (start 134.8958 69.0662) (end 134.8958 47.2658) (width 0.5) (layer F.Cu) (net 2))
 (segment (start 134.8958 47.2658) (end 133.35 45.72) (width 0.5) (layer F.Cu) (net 2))
 (segment (start 133.35 45.72) (end 131.8497 45.72) (width 0.5) (layer F.Cu) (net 2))
 (segment (start 117.042 32.258) (end 118.4723 32.258) (width 0.5) (layer F.Cu) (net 2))
 (segment (start 131.8497 45.72) (end 131.8497 45.6354) (width 0.5) (layer F.Cu) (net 2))
 (segment (start 131.8497 45.6354) (end 118.4723 32.258) (width 0.5) (layer F.Cu) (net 2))
 (segment (start 57.15 41.8153) (end 56.7827 41.8153) (width 0.25) (layer B.Cu) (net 21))
 (segment (start 56.7827 41.8153) (end 54.8318 43.7662) (width 0.25) (layer B.Cu) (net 21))
 (segment (start 54.8318 43.7662) (end 54.8318 73.9264) (width 0.25) (layer B.Cu) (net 21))
 (segment (start 54.8318 73.9264) (end 55.8873 74.9819) (width 0.25) (layer B.Cu) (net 21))
 (segment (start 55.8873 74.9819) (end 58.4535 74.9819) (width 0.25) (layer B.Cu) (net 21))
 (segment (start 58.4535 74.9819) (end 59.0137 74.4217) (width 0.25) (layer B.Cu) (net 21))
 (segment (start 59.0137 74.4217) (end 59.0137 68.2037) (width 0.25) (layer B.Cu) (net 21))
 (segment (start 59.0137 68.2037) (end 57.5173 66.7073) (width 0.25) (layer B.Cu) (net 21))
 (segment (start 57.5173 66.7073) (end 57.15 66.7073) (width 0.25) (layer B.Cu) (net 21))
 (segment (start 57.15 40.64) (end 57.15 41.8153) (width 0.25) (layer B.Cu) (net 21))
 (segment (start 57.15 65.532) (end 57.15 66.7073) (width 0.25) (layer B.Cu) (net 21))
 (segment (start 111.962 57.658) (end 113.7402 59.4362) (width 0.25) (layer B.Cu) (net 21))
 (segment (start 113.7402 59.4362) (end 117.7491 59.4362) (width 0.25) (layer B.Cu) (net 21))
 (segment (start 117.7491 59.4362) (end 119.9576 57.2277) (width 0.25) (layer B.Cu) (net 21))
 (segment (start 119.9576 57.2277) (end 119.9576 55.397) (width 0.25) (layer B.Cu) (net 21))
 (segment (start 119.9576 55.397) (end 119.9577 55.397) (width 0.25) (layer B.Cu) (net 21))
 (segment (start 119.9577 55.397) (end 132.1747 43.18) (width 0.25) (layer B.Cu) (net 21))
 (segment (start 133.35 68.072) (end 133.35 66.8967) (width 0.25) (layer B.Cu) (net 21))
 (segment (start 133.35 66.8967) (end 132.9827 66.8967) (width 0.25) (layer B.Cu) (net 21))
 (segment (start 132.9827 66.8967) (end 131.4923 65.4063) (width 0.25) (layer B.Cu) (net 21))
 (segment (start 131.4923 65.4063) (end 131.4923 53.3364) (width 0.25) (layer B.Cu) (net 21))
 (segment (start 131.4923 53.3364) (end 134.7654 50.0633) (width 0.25) (layer B.Cu) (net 21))
 (segment (start 134.7654 50.0633) (end 134.7654 44.5954) (width 0.25) (layer B.Cu) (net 21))
 (segment (start 134.7654 44.5954) (end 133.35 43.18) (width 0.25) (layer B.Cu) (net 21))
 (segment (start 133.35 43.18) (end 132.1747 43.18) (width 0.25) (layer B.Cu) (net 21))
 (segment (start 57.15 40.64) (end 94.944 40.64) (width 0.25) (layer F.Cu) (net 21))
 (segment (start 94.944 40.64) (end 111.962 57.658) (width 0.25) (layer F.Cu) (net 21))
 (segment (start 57.15 43.18) (end 57.15 44.3553) (width 0.25) (layer B.Cu) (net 18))
 (segment (start 57.15 68.072) (end 58.5634 69.4854) (width 0.25) (layer B.Cu) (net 18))
 (segment (start 58.5634 69.4854) (end 58.5634 74.2351) (width 0.25) (layer B.Cu) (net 18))
 (segment (start 58.5634 74.2351) (end 58.2669 74.5316) (width 0.25) (layer B.Cu) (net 18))
 (segment (start 58.2669 74.5316) (end 56.0739 74.5316) (width 0.25) (layer B.Cu) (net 18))
 (segment (start 56.0739 74.5316) (end 55.2821 73.7398) (width 0.25) (layer B.Cu) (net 18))
 (segment (start 55.2821 73.7398) (end 55.2821 45.8558) (width 0.25) (layer B.Cu) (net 18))
 (segment (start 55.2821 45.8558) (end 56.7826 44.3553) (width 0.25) (layer B.Cu) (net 18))
 (segment (start 56.7826 44.3553) (end 57.15 44.3553) (width 0.25) (layer B.Cu) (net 18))
 (segment (start 104.342 57.658) (end 105.4498 56.5502) (width 0.25) (layer B.Cu) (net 18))
 (segment (start 105.4498 56.5502) (end 112.4683 56.5502) (width 0.25) (layer B.Cu) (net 18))
 (segment (start 112.4683 56.5502) (end 113.232 57.3139) (width 0.25) (layer B.Cu) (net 18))
 (segment (start 113.232 57.3139) (end 113.232 58.0401) (width 0.25) (layer B.Cu) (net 18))
 (segment (start 113.232 58.0401) (end 114.1778 58.9859) (width 0.25) (layer B.Cu) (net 18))
 (segment (start 114.1778 58.9859) (end 117.5625 58.9859) (width 0.25) (layer B.Cu) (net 18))
 (segment (start 117.5625 58.9859) (end 118.8991 57.6493) (width 0.25) (layer B.Cu) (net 18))
 (segment (start 118.8991 57.6493) (end 118.8991 55.752) (width 0.25) (layer B.Cu) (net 18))
 (segment (start 118.8991 55.752) (end 132.8358 41.8153) (width 0.25) (layer B.Cu) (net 18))
 (segment (start 132.8358 41.8153) (end 133.35 41.8153) (width 0.25) (layer B.Cu) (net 18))
 (segment (start 57.15 43.18) (end 89.864 43.18) (width 0.25) (layer F.Cu) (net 18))
 (segment (start 89.864 43.18) (end 104.342 57.658) (width 0.25) (layer F.Cu) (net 18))
 (segment (start 133.35 64.3567) (end 132.9827 64.3567) (width 0.25) (layer B.Cu) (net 18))
 (segment (start 132.9827 64.3567) (end 131.9746 63.3486) (width 0.25) (layer B.Cu) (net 18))
 (segment (start 131.9746 63.3486) (end 131.9746 53.7339) (width 0.25) (layer B.Cu) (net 18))
 (segment (start 131.9746 53.7339) (end 135.2158 50.4927) (width 0.25) (layer B.Cu) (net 18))
 (segment (start 135.2158 50.4927) (end 135.2158 43.3138) (width 0.25) (layer B.Cu) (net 18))
 (segment (start 135.2158 43.3138) (end 133.7173 41.8153) (width 0.25) (layer B.Cu) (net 18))
 (segment (start 133.7173 41.8153) (end 133.35 41.8153) (width 0.25) (layer B.Cu) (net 18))
 (segment (start 133.35 40.64) (end 133.35 41.8153) (width 0.25) (layer B.Cu) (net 18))
 (segment (start 133.35 65.532) (end 133.35 64.3567) (width 0.25) (layer B.Cu) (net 18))
 (segment (start 55.7746 56.5229) (end 55.7746 47.0954) (width 0.25) (layer B.Cu) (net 16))
 (segment (start 55.7746 47.0954) (end 57.15 45.72) (width 0.25) (layer B.Cu) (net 16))
 (segment (start 57.15 69.4367) (end 56.7827 69.4367) (width 0.25) (layer B.Cu) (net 16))
 (segment (start 56.7827 69.4367) (end 55.7746 68.4286) (width 0.25) (layer B.Cu) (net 16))
 (segment (start 55.7746 68.4286) (end 55.7746 56.5229) (width 0.25) (layer B.Cu) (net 16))
 (segment (start 55.7746 56.5229) (end 90.5069 56.5229) (width 0.25) (layer B.Cu) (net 16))
 (segment (start 90.5069 56.5229) (end 91.642 57.658) (width 0.25) (layer B.Cu) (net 16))
 (segment (start 57.15 70.612) (end 57.15 69.4367) (width 0.25) (layer B.Cu) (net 16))
 (segment (start 133.35 62.992) (end 132.1747 62.992) (width 0.25) (layer F.Cu) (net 16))
 (segment (start 132.1747 62.992) (end 125.862 69.3047) (width 0.25) (layer F.Cu) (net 16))
 (segment (start 125.862 69.3047) (end 118.5803 69.3047) (width 0.25) (layer F.Cu) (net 16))
 (segment (start 118.5803 69.3047) (end 117.6946 68.419) (width 0.25) (layer F.Cu) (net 16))
 (segment (start 117.6946 68.419) (end 117.6946 62.143) (width 0.25) (layer F.Cu) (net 16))
 (segment (start 117.6946 62.143) (end 115.5579 60.0063) (width 0.25) (layer F.Cu) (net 16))
 (segment (start 115.5579 60.0063) (end 105.1068 60.0063) (width 0.25) (layer F.Cu) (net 16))
 (segment (start 105.1068 60.0063) (end 103.2134 58.1129) (width 0.25) (layer F.Cu) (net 16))
 (segment (start 103.2134 58.1129) (end 103.2134 57.1663) (width 0.25) (layer F.Cu) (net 16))
 (segment (start 103.2134 57.1663) (end 102.3488 56.3017) (width 0.25) (layer F.Cu) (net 16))
 (segment (start 102.3488 56.3017) (end 92.9983 56.3017) (width 0.25) (layer F.Cu) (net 16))
 (segment (start 92.9983 56.3017) (end 91.642 57.658) (width 0.25) (layer F.Cu) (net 16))
 (segment (start 133.35 38.1) (end 133.35 39.2753) (width 0.25) (layer B.Cu) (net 16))
 (segment (start 133.35 62.992) (end 135.6946 60.6474) (width 0.25) (layer B.Cu) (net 16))
 (segment (start 135.6946 60.6474) (end 135.6946 41.2526) (width 0.25) (layer B.Cu) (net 16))
 (segment (start 135.6946 41.2526) (end 133.7173 39.2753) (width 0.25) (layer B.Cu) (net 16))
 (segment (start 133.7173 39.2753) (end 133.35 39.2753) (width 0.25) (layer B.Cu) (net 16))
 (segment (start 84.022 41.91) (end 65.0003 41.91) (width 0.5) (layer B.Cu) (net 4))
 (segment (start 65.0003 41.91) (end 58.6503 48.26) (width 0.5) (layer B.Cu) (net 4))
 (segment (start 101.802 55.2527) (end 88.4593 41.91) (width 0.5) (layer B.Cu) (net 4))
 (segment (start 88.4593 41.91) (end 84.022 41.91) (width 0.5) (layer B.Cu) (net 4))
 (segment (start 84.022 32.258) (end 84.022 41.91) (width 0.5) (layer B.Cu) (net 4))
 (segment (start 57.15 48.26) (end 58.6503 48.26) (width 0.5) (layer B.Cu) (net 4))
 (segment (start 120.016 60.6961) (end 120.016 67.008) (width 0.5) (layer F.Cu) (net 4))
 (segment (start 117.042 57.658) (end 120.016 60.632) (width 0.5) (layer F.Cu) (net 4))
 (segment (start 120.016 60.632) (end 120.016 60.6961) (width 0.5) (layer F.Cu) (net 4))
 (segment (start 131.8497 60.452) (end 131.6056 60.6961) (width 0.5) (layer F.Cu) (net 4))
 (segment (start 131.6056 60.6961) (end 120.016 60.6961) (width 0.5) (layer F.Cu) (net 4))
 (segment (start 133.35 60.452) (end 131.8497 60.452) (width 0.5) (layer F.Cu) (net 4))
 (segment (start 115.316 70.008) (end 118.316 67.008) (width 0.5) (layer B.Cu) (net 4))
 (segment (start 118.316 67.008) (end 120.016 67.008) (width 0.5) (layer B.Cu) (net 4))
 (segment (start 117.042 55.2527) (end 117.042 51.868) (width 0.5) (layer B.Cu) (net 4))
 (segment (start 117.042 51.868) (end 133.35 35.56) (width 0.5) (layer B.Cu) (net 4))
 (segment (start 117.042 57.658) (end 117.042 55.2527) (width 0.5) (layer B.Cu) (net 4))
 (segment (start 117.042 55.2527) (end 101.802 55.2527) (width 0.5) (layer B.Cu) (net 4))
 (segment (start 101.802 55.2527) (end 101.802 57.658) (width 0.5) (layer B.Cu) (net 4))
 (segment (start 95.8897 64.5366) (end 96.9603 63.466) (width 0.5) (layer F.Cu) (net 4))
 (segment (start 96.9603 63.466) (end 96.9603 62.4997) (width 0.5) (layer F.Cu) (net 4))
 (segment (start 96.9603 62.4997) (end 101.802 57.658) (width 0.5) (layer F.Cu) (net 4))
 (segment (start 92.7783 67.648) (end 95.8897 64.5366) (width 0.5) (layer F.Cu) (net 4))
 (segment (start 89.662 72.5405) (end 91.3799 74.2584) (width 0.5) (layer F.Cu) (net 4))
 (segment (start 91.3799 74.2584) (end 100.3359 74.2584) (width 0.5) (layer F.Cu) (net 4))
 (segment (start 100.3359 74.2584) (end 100.7321 73.8622) (width 0.5) (layer F.Cu) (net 4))
 (segment (start 100.7321 73.8622) (end 100.7321 69.3791) (width 0.5) (layer F.Cu) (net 4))
 (segment (start 100.7321 69.3791) (end 95.8897 64.5366) (width 0.5) (layer F.Cu) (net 4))
 (segment (start 86.548 72.5405) (end 89.662 72.5405) (width 0.5) (layer F.Cu) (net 4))
 (segment (start 84.582 72.5405) (end 86.548 72.5405) (width 0.5) (layer F.Cu) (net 4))
 (segment (start 86.548 72.5405) (end 86.548 67.648) (width 0.5) (layer F.Cu) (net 4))
 (segment (start 58.6503 73.152) (end 58.8765 72.9258) (width 0.5) (layer F.Cu) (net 4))
 (segment (start 58.8765 72.9258) (end 65.3354 72.9258) (width 0.5) (layer F.Cu) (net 4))
 (segment (start 65.3354 72.9258) (end 66.6823 74.2727) (width 0.5) (layer F.Cu) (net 4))
 (segment (start 66.6823 74.2727) (end 82.8498 74.2727) (width 0.5) (layer F.Cu) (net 4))
 (segment (start 82.8498 74.2727) (end 84.582 72.5405) (width 0.5) (layer F.Cu) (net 4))
 (segment (start 91.628 67.648) (end 92.7783 67.648) (width 0.5) (layer F.Cu) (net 4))
 (segment (start 57.15 73.152) (end 58.6503 73.152) (width 0.5) (layer F.Cu) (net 4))
 (segment (start 99.06 71.628) (end 97.4197 71.628) (width 0.5) (layer F.Cu) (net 6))
 (segment (start 89.728 70.6495) (end 89.662 70.7155) (width 0.5) (layer F.Cu) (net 6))
 (segment (start 89.728 67.648) (end 89.728 70.6495) (width 0.5) (layer F.Cu) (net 6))
 (segment (start 97.4197 71.628) (end 96.4412 70.6495) (width 0.5) (layer F.Cu) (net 6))
 (segment (start 96.4412 70.6495) (end 89.728 70.6495) (width 0.5) (layer F.Cu) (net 6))
 (segment (start 84.648 67.648) (end 83.4977 67.648) (width 0.5) (layer F.Cu) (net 3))
 (segment (start 83.4838 68.9556) (end 83.4838 69.6173) (width 0.5) (layer F.Cu) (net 3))
 (segment (start 83.4838 69.6173) (end 84.582 70.7155) (width 0.5) (layer F.Cu) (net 3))
 (segment (start 83.4977 67.648) (end 83.4977 68.9417) (width 0.5) (layer F.Cu) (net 3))
 (segment (start 83.4977 68.9417) (end 83.4838 68.9556) (width 0.5) (layer F.Cu) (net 3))
 (segment (start 72.7603 71.628) (end 75.4327 68.9556) (width 0.5) (layer F.Cu) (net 3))
 (segment (start 75.4327 68.9556) (end 83.4838 68.9556) (width 0.5) (layer F.Cu) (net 3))
 (segment (start 71.12 71.628) (end 72.7603 71.628) (width 0.5) (layer F.Cu) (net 3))
 (segment (start 90.7815 64.4158) (end 90.7815 63.246) (width 0.5) (layer F.Cu) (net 5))
 (segment (start 90.678 65.448) (end 90.7815 65.3445) (width 0.5) (layer F.Cu) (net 5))
 (segment (start 90.7815 65.3445) (end 90.7815 64.4158) (width 0.5) (layer F.Cu) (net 5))
 (segment (start 96.722 57.658) (end 96.722 60.8831) (width 0.5) (layer F.Cu) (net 5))
 (segment (start 96.722 60.8831) (end 93.1893 64.4158) (width 0.5) (layer F.Cu) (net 5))
 (segment (start 93.1893 64.4158) (end 90.7815 64.4158) (width 0.5) (layer F.Cu) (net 5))
 (segment (start 85.4945 63.246) (end 89.0762 63.246) (width 0.5) (layer F.Cu) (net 1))
 (segment (start 99.262 57.658) (end 93.674 63.246) (width 0.5) (layer B.Cu) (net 1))
 (segment (start 93.674 63.246) (end 89.0762 63.246) (width 0.5) (layer B.Cu) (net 1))
 (segment (start 85.598 64.0977) (end 85.4945 63.9942) (width 0.5) (layer F.Cu) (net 1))
 (segment (start 85.4945 63.9942) (end 85.4945 63.246) (width 0.5) (layer F.Cu) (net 1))
 (segment (start 85.598 65.448) (end 85.598 64.0977) (width 0.5) (layer F.Cu) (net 1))
 (via (at 89.0762 63.246) (size 1.6) (drill 0.8) (layers F.Cu B.Cu) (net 1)))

